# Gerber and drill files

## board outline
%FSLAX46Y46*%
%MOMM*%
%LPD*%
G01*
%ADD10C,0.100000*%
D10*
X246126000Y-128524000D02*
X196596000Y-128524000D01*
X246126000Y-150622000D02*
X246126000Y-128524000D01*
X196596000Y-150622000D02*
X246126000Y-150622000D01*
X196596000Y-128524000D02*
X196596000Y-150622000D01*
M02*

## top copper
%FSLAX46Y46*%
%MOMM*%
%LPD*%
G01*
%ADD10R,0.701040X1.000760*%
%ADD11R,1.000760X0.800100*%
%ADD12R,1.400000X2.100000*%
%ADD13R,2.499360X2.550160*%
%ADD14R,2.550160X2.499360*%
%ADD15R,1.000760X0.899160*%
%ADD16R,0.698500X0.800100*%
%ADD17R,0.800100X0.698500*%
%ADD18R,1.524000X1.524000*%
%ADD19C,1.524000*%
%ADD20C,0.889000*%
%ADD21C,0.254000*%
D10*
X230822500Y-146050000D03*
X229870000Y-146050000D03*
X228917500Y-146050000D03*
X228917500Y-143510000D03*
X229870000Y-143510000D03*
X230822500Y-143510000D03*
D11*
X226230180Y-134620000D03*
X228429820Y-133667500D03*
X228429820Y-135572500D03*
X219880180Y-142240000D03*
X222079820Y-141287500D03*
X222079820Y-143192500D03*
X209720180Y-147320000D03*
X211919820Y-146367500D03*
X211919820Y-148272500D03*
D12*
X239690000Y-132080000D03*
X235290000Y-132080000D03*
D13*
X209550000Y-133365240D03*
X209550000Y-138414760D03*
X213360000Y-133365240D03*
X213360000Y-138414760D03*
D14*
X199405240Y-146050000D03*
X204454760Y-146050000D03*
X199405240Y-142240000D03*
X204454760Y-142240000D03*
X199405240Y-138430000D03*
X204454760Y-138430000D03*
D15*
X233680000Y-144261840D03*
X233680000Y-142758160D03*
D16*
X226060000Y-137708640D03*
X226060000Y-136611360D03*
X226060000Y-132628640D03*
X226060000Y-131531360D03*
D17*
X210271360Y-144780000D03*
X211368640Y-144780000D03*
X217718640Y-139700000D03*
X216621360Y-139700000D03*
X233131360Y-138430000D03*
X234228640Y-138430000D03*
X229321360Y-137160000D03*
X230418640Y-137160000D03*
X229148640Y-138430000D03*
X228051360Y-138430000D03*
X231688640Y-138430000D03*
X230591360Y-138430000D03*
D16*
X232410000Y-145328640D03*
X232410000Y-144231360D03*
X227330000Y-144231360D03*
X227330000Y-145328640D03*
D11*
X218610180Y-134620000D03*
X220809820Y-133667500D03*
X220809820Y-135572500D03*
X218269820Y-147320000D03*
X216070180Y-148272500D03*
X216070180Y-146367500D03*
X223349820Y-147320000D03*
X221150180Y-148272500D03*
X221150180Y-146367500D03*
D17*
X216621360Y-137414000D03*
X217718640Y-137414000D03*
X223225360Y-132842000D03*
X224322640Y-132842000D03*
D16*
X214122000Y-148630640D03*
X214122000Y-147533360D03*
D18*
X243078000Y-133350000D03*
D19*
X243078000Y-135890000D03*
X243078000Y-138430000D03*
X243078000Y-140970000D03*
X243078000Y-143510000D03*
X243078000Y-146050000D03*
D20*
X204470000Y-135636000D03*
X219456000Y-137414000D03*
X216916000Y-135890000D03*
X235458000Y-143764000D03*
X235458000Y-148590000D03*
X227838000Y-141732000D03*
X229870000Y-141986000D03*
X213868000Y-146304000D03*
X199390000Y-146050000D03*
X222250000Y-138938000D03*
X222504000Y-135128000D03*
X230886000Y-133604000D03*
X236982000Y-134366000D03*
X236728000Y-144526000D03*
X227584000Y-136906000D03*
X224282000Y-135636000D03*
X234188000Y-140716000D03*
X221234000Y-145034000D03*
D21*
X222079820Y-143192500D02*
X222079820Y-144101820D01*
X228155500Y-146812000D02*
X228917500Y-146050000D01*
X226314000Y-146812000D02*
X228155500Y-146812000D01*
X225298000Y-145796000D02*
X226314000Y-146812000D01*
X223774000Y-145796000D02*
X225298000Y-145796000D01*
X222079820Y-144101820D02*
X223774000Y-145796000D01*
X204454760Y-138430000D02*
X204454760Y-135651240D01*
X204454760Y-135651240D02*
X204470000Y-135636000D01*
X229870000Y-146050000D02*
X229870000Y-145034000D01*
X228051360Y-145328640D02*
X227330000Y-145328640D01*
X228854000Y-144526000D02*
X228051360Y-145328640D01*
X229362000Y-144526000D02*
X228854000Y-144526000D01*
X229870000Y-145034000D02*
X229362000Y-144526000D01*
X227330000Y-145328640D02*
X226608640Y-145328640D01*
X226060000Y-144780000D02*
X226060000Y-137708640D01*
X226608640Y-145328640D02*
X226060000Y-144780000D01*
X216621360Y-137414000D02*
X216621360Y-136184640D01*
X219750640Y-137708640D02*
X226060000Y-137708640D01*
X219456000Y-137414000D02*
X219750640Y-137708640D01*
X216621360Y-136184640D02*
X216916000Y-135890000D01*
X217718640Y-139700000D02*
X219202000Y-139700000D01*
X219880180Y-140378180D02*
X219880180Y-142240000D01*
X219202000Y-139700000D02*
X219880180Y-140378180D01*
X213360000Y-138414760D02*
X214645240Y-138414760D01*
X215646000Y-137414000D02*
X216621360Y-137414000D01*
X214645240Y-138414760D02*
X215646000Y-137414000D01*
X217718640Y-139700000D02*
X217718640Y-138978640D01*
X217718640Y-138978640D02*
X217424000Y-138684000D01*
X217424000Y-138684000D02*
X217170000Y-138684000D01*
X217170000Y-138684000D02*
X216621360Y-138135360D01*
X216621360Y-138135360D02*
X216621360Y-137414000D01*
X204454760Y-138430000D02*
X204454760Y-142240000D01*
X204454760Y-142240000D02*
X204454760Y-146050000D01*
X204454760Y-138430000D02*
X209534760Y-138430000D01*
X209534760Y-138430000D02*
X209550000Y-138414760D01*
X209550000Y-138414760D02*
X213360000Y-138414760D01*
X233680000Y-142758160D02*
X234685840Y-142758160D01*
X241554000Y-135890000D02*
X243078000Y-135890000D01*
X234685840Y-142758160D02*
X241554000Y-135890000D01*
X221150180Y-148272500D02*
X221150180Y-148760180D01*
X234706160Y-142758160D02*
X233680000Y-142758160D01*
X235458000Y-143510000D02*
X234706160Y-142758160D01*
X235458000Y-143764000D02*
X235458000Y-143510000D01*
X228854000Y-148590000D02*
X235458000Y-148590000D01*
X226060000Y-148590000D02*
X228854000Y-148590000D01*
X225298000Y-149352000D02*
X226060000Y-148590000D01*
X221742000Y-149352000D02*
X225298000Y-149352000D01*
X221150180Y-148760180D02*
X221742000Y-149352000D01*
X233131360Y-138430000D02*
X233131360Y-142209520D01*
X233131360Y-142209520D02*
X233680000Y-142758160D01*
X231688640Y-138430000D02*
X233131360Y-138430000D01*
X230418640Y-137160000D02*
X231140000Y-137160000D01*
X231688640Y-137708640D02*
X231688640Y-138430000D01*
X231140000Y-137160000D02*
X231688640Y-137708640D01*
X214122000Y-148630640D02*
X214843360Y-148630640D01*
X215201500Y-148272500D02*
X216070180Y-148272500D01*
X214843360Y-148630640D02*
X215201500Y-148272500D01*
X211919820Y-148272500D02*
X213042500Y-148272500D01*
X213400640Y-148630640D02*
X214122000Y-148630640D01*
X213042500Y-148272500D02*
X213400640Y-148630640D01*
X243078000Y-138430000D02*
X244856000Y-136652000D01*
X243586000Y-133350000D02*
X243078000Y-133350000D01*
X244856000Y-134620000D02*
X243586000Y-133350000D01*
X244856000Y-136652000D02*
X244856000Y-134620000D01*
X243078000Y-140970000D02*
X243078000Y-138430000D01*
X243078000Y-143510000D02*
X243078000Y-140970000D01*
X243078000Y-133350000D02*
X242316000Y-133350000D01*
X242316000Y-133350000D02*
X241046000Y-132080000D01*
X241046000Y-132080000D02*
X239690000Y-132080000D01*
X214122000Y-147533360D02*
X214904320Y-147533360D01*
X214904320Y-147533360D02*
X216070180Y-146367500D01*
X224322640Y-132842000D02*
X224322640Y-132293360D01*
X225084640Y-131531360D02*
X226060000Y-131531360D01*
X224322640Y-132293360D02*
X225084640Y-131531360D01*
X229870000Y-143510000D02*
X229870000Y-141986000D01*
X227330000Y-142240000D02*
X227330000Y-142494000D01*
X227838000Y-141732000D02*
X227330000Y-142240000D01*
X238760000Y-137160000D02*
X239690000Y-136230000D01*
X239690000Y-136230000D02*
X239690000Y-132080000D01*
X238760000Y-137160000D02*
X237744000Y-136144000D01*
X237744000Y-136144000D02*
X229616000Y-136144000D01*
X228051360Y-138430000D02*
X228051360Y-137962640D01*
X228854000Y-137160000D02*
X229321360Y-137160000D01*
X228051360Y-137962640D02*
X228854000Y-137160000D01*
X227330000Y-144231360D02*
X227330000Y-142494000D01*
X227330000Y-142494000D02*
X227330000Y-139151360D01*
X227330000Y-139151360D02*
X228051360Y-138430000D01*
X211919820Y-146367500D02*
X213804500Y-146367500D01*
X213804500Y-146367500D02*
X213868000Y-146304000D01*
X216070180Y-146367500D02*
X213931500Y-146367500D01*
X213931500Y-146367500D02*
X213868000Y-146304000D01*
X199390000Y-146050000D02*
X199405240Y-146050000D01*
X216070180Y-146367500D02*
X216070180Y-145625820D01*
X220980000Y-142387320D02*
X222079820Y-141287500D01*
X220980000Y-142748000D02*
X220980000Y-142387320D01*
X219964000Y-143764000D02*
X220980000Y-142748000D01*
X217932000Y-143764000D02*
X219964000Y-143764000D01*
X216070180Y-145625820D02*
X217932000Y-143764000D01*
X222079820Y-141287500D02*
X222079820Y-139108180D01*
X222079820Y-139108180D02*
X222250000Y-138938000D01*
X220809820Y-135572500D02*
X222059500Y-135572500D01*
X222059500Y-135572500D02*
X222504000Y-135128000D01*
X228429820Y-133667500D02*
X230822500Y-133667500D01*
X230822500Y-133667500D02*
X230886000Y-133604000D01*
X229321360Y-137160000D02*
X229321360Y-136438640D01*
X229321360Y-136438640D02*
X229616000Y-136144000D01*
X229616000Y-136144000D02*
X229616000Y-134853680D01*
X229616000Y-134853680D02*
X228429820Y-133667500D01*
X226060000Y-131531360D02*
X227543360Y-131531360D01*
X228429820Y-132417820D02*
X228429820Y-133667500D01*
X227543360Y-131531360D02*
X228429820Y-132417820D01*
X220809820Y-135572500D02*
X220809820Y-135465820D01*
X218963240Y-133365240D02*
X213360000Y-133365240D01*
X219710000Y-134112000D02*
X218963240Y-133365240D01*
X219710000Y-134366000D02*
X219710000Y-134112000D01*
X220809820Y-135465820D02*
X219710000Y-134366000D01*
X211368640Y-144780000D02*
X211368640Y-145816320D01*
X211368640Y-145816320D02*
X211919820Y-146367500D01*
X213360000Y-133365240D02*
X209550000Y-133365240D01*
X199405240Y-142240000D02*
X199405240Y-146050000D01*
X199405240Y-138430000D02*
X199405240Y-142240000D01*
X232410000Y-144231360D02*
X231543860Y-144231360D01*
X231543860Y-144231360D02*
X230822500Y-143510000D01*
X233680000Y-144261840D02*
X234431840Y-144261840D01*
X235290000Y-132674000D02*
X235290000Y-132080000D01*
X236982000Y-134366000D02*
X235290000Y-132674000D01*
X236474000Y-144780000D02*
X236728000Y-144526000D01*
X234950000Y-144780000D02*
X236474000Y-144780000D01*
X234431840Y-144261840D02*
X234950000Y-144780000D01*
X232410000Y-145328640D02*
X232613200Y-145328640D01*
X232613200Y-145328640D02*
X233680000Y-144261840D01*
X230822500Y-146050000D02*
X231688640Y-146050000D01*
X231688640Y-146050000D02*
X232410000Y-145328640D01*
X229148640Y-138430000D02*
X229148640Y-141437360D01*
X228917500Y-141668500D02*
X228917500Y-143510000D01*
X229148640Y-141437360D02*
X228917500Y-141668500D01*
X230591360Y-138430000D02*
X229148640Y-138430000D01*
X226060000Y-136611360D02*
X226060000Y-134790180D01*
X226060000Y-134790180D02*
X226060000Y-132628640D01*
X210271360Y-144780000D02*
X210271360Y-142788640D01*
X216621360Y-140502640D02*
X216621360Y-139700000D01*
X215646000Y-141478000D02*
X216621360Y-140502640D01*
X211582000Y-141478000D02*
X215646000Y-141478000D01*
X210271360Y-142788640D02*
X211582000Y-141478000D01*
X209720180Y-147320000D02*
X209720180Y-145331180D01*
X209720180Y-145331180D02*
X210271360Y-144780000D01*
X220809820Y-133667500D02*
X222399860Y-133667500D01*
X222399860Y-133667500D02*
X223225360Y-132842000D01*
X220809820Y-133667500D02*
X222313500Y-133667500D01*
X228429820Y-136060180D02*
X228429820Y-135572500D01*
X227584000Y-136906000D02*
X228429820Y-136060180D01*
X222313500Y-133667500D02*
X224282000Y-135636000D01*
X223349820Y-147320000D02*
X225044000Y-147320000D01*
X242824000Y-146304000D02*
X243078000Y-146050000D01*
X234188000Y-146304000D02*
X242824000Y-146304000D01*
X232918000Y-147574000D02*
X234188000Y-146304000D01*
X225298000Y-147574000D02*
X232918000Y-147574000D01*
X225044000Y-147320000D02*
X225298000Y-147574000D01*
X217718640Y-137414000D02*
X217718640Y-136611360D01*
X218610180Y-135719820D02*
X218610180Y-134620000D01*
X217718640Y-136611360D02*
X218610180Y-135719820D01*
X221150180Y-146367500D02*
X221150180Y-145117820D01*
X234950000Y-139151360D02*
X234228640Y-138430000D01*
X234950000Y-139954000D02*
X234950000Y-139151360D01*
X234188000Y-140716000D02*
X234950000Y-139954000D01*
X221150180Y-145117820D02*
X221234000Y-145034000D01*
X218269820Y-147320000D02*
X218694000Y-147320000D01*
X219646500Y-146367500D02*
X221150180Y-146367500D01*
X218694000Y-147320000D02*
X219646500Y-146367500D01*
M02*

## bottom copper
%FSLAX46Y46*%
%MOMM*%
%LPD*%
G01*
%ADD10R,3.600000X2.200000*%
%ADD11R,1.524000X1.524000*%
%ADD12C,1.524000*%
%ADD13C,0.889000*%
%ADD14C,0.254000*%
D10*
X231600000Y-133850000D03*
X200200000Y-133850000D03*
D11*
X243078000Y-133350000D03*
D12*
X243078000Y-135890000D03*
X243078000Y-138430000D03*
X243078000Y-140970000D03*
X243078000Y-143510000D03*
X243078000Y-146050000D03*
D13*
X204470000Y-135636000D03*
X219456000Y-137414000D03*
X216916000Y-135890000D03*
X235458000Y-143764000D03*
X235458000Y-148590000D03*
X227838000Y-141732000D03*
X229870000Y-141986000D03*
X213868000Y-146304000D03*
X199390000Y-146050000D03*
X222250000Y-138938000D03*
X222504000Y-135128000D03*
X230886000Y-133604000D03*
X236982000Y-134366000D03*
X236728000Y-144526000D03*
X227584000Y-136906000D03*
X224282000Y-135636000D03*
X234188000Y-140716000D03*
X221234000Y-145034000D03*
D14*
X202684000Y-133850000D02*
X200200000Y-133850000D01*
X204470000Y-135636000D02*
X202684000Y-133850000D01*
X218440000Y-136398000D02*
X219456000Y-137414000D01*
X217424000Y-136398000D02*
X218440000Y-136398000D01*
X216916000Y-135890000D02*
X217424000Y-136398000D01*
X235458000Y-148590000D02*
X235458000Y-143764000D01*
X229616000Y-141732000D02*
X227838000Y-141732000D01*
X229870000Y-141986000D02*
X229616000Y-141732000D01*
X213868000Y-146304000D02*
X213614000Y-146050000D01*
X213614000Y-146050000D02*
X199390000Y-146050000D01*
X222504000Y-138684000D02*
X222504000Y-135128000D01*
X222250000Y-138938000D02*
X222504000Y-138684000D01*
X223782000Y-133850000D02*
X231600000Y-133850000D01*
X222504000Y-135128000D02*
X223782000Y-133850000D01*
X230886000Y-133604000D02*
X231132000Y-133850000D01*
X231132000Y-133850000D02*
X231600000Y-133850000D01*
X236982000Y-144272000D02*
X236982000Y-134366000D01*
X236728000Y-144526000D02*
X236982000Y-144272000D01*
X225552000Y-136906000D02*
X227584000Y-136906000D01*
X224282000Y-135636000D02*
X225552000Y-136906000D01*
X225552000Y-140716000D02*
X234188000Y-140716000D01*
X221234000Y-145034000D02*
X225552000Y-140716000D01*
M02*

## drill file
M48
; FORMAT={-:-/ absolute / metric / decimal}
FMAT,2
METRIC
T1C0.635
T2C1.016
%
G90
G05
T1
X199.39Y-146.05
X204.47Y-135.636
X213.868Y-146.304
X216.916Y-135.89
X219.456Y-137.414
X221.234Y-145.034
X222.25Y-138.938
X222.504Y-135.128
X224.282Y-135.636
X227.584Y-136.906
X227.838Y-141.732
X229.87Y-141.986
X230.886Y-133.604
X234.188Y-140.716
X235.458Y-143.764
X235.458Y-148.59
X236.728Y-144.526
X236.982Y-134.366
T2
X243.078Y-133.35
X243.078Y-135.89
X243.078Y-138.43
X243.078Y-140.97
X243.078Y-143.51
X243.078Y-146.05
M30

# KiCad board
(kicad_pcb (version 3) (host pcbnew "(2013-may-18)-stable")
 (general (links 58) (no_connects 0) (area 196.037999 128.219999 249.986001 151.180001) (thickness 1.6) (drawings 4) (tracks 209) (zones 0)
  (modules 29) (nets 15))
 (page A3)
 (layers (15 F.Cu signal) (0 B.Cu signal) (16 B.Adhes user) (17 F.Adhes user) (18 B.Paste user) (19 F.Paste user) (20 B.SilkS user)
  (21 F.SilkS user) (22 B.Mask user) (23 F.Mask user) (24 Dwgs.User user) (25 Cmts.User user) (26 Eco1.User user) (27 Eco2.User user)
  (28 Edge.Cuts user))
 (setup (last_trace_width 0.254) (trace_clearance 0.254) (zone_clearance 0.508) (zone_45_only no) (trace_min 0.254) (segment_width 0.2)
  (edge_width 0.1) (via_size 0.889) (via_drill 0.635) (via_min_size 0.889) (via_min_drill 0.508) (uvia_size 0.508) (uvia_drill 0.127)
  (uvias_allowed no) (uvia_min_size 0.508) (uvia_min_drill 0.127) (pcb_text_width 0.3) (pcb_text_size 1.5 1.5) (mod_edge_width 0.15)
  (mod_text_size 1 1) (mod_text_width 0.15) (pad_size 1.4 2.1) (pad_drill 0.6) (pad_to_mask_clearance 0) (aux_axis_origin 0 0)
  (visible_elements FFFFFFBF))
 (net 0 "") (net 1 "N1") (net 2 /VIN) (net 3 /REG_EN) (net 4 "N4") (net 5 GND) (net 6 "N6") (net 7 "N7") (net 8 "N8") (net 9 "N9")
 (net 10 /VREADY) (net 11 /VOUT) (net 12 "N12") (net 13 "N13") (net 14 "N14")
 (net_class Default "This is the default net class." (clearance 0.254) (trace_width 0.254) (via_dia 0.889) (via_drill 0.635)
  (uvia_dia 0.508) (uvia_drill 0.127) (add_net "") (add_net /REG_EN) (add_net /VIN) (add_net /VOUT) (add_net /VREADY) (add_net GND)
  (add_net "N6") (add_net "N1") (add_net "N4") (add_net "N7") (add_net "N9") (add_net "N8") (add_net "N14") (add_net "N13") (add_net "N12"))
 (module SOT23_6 (layer F.Cu) (at 229.87 144.78 180)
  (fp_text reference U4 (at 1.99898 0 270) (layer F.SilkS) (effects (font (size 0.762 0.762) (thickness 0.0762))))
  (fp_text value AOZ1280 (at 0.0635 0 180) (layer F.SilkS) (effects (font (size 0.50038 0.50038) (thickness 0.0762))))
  (pad 6 smd rect (at -0.9525 -1.27 180) (size 0.70104 1.00076) (layers F.Cu F.Paste F.Mask) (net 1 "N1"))
  (pad 5 smd rect (at 0 -1.27 180) (size 0.70104 1.00076) (layers F.Cu F.Paste F.Mask) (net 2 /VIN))
  (pad 4 smd rect (at 0.9525 -1.27 180) (size 0.70104 1.00076) (layers F.Cu F.Paste F.Mask) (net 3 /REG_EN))
  (pad 3 smd rect (at 0.9525 1.27 180) (size 0.70104 1.00076) (layers F.Cu F.Paste F.Mask) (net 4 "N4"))
  (pad 2 smd rect (at 0 1.27 180) (size 0.70104 1.00076) (layers F.Cu F.Paste F.Mask) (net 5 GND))
  (pad 1 smd rect (at -0.9525 1.27 180) (size 0.70104 1.00076) (layers F.Cu F.Paste F.Mask) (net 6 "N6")))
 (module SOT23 (layer F.Cu) (at 227.33 134.62 90)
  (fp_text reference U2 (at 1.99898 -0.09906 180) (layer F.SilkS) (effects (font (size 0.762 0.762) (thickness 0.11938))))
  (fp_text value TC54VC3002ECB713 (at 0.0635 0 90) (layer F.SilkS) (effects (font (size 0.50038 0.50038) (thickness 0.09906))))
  (pad 3 smd rect (at 0 -1.09982 90) (size 0.8001 1.00076) (layers F.Cu F.Paste F.Mask) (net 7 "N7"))
  (pad 2 smd rect (at 0.9525 1.09982 90) (size 0.8001 1.00076) (layers F.Cu F.Paste F.Mask) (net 5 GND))
  (pad 1 smd rect (at -0.9525 1.09982 90) (size 0.8001 1.00076) (layers F.Cu F.Paste F.Mask) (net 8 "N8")))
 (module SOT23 (layer F.Cu) (at 220.98 142.24 90)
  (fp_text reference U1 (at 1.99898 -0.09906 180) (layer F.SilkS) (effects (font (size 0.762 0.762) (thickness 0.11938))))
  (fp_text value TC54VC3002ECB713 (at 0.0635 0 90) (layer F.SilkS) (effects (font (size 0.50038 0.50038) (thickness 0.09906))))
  (pad 3 smd rect (at 0 -1.09982 90) (size 0.8001 1.00076) (layers F.Cu F.Paste F.Mask) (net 2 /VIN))
  (pad 2 smd rect (at 0.9525 1.09982 90) (size 0.8001 1.00076) (layers F.Cu F.Paste F.Mask) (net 5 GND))
  (pad 1 smd rect (at -0.9525 1.09982 90) (size 0.8001 1.00076) (layers F.Cu F.Paste F.Mask) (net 3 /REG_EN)))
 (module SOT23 (layer F.Cu) (at 210.82 147.32 90)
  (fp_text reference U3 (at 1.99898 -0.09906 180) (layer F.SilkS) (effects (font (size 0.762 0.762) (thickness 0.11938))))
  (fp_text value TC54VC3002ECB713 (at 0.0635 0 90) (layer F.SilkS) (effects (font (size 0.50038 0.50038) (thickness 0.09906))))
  (pad 3 smd rect (at 0 -1.09982 90) (size 0.8001 1.00076) (layers F.Cu F.Paste F.Mask) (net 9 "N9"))
  (pad 2 smd rect (at 0.9525 1.09982 90) (size 0.8001 1.00076) (layers F.Cu F.Paste F.Mask) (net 5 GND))
  (pad 1 smd rect (at -0.9525 1.09982 90) (size 0.8001 1.00076) (layers F.Cu F.Paste F.Mask) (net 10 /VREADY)))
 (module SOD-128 (layer F.Cu) (at 237.49 132.08 180)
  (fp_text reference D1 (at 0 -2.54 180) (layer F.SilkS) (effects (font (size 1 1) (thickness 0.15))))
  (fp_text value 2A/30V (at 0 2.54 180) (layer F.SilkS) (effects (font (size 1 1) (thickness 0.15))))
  (pad 1 smd rect (at -2.2 0 180) (size 1.4 2.1) (layers F.Cu F.Paste F.Mask) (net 5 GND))
  (pad 2 smd rect (at 2.2 0 180) (size 1.4 2.1) (layers F.Cu F.Paste F.Mask) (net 1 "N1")))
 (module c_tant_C (layer F.Cu) (at 209.55 135.89 90)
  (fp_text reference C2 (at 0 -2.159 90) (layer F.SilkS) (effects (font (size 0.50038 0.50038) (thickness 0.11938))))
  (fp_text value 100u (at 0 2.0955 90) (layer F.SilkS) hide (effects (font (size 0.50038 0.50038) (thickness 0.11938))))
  (pad 1 smd rect (at 2.52476 0 90) (size 2.55016 2.49936) (layers F.Cu F.Paste F.Mask) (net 5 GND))
  (pad 2 smd rect (at -2.52476 0 90) (size 2.55016 2.49936) (layers F.Cu F.Paste F.Mask) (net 2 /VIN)))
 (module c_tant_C (layer F.Cu) (at 213.36 135.89 90)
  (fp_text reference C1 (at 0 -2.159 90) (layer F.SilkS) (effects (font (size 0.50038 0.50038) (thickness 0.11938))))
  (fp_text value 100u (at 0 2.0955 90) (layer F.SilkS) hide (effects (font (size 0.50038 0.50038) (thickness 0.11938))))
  (pad 1 smd rect (at 2.52476 0 90) (size 2.55016 2.49936) (layers F.Cu F.Paste F.Mask) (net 5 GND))
  (pad 2 smd rect (at -2.52476 0 90) (size 2.55016 2.49936) (layers F.Cu F.Paste F.Mask) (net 2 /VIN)))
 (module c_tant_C (layer F.Cu) (at 201.93 146.05 180)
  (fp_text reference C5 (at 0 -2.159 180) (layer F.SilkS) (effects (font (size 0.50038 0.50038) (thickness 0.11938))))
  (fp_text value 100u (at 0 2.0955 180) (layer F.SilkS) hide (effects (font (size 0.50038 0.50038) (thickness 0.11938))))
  (pad 1 smd rect (at 2.52476 0 180) (size 2.55016 2.49936) (layers F.Cu F.Paste F.Mask) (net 5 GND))
  (pad 2 smd rect (at -2.52476 0 180) (size 2.55016 2.49936) (layers F.Cu F.Paste F.Mask) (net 2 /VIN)))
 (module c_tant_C (layer F.Cu) (at 201.93 142.24 180)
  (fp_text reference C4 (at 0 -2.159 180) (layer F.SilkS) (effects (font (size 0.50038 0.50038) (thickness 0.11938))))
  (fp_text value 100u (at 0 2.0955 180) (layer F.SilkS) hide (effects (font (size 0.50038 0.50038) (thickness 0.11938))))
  (pad 1 smd rect (at 2.52476 0 180) (size 2.55016 2.49936) (layers F.Cu F.Paste F.Mask) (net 5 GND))
  (pad 2 smd rect (at -2.52476 0 180) (size 2.55016 2.49936) (layers F.Cu F.Paste F.Mask) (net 2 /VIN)))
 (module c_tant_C (layer F.Cu) (at 201.93 138.43 180)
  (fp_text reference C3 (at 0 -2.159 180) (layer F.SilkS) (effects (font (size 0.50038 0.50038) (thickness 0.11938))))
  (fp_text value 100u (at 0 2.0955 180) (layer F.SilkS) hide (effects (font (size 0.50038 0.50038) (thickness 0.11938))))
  (pad 1 smd rect (at 2.52476 0 180) (size 2.55016 2.49936) (layers F.Cu F.Paste F.Mask) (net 5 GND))
  (pad 2 smd rect (at -2.52476 0 180) (size 2.55016 2.49936) (layers F.Cu F.Paste F.Mask) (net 2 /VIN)))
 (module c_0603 (layer F.Cu) (at 233.68 143.51 270)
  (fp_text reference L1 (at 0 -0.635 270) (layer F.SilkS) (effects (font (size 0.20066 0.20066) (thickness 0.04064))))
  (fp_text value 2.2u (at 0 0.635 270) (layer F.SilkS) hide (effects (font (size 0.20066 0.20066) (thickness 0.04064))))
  (pad 1 smd rect (at 0.75184 0 270) (size 0.89916 1.00076) (layers F.Cu F.Paste F.Mask) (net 1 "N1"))
  (pad 2 smd rect (at -0.75184 0 270) (size 0.89916 1.00076) (layers F.Cu F.Paste F.Mask) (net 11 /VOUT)))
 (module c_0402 (layer F.Cu) (at 226.06 137.16 270)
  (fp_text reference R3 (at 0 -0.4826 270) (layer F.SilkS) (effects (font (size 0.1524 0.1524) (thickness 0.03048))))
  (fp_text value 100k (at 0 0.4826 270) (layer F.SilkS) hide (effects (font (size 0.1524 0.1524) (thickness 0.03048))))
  (pad 1 smd rect (at 0.54864 0 270) (size 0.8001 0.6985) (layers F.Cu F.Paste F.Mask) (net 2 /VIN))
  (pad 2 smd rect (at -0.54864 0 270) (size 0.8001 0.6985) (layers F.Cu F.Paste F.Mask) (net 7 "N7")))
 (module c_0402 (layer F.Cu) (at 226.06 132.08 270)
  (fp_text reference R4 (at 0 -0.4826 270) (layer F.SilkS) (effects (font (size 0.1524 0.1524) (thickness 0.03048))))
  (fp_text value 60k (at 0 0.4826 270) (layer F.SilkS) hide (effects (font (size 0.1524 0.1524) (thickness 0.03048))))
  (pad 1 smd rect (at 0.54864 0 270) (size 0.8001 0.6985) (layers F.Cu F.Paste F.Mask) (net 7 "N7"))
  (pad 2 smd rect (at -0.54864 0 270) (size 0.8001 0.6985) (layers F.Cu F.Paste F.Mask) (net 5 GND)))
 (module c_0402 (layer F.Cu) (at 210.82 144.78 180)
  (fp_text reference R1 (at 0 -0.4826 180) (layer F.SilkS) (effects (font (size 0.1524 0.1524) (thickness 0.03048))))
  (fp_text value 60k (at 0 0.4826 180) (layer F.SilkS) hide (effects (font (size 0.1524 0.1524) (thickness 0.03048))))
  (pad 1 smd rect (at 0.54864 0 180) (size 0.8001 0.6985) (layers F.Cu F.Paste F.Mask) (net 9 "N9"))
  (pad 2 smd rect (at -0.54864 0 180) (size 0.8001 0.6985) (layers F.Cu F.Paste F.Mask) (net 5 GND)))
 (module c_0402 (layer F.Cu) (at 217.17 139.7)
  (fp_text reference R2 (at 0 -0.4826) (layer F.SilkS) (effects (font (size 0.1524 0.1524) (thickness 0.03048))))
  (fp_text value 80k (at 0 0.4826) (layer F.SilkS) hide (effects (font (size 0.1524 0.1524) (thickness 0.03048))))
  (pad 1 smd rect (at 0.54864 0) (size 0.8001 0.6985) (layers F.Cu F.Paste F.Mask) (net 2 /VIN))
  (pad 2 smd rect (at -0.54864 0) (size 0.8001 0.6985) (layers F.Cu F.Paste F.Mask) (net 9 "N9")))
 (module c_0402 (layer F.Cu) (at 233.68 138.43 180)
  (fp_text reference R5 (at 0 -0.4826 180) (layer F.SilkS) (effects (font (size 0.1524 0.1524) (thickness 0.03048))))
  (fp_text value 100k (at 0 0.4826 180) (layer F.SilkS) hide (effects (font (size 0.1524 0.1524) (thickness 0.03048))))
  (pad 1 smd rect (at 0.54864 0 180) (size 0.8001 0.6985) (layers F.Cu F.Paste F.Mask) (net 11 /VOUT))
  (pad 2 smd rect (at -0.54864 0 180) (size 0.8001 0.6985) (layers F.Cu F.Paste F.Mask) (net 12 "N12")))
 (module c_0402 (layer F.Cu) (at 229.87 137.16 180)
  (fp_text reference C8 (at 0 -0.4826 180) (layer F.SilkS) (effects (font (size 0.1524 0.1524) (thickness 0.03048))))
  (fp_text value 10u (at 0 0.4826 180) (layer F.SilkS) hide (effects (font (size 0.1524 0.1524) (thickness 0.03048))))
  (pad 1 smd rect (at 0.54864 0 180) (size 0.8001 0.6985) (layers F.Cu F.Paste F.Mask) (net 5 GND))
  (pad 2 smd rect (at -0.54864 0 180) (size 0.8001 0.6985) (layers F.Cu F.Paste F.Mask) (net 11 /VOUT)))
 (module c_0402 (layer F.Cu) (at 228.6 138.43)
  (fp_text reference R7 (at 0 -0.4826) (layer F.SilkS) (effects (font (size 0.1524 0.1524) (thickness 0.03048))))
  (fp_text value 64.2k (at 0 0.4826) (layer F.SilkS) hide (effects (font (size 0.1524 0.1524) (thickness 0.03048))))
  (pad 1 smd rect (at 0.54864 0) (size 0.8001 0.6985) (layers F.Cu F.Paste F.Mask) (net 4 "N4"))
  (pad 2 smd rect (at -0.54864 0) (size 0.8001 0.6985) (layers F.Cu F.Paste F.Mask) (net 5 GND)))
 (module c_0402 (layer F.Cu) (at 231.14 138.43)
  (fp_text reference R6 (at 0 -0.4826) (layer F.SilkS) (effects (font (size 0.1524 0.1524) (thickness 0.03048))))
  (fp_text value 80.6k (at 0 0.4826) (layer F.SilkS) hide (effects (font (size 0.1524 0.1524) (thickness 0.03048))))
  (pad 1 smd rect (at 0.54864 0) (size 0.8001 0.6985) (layers F.Cu F.Paste F.Mask) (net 11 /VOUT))
  (pad 2 smd rect (at -0.54864 0) (size 0.8001 0.6985) (layers F.Cu F.Paste F.Mask) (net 4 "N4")))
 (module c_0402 (layer F.Cu) (at 232.41 144.78 270)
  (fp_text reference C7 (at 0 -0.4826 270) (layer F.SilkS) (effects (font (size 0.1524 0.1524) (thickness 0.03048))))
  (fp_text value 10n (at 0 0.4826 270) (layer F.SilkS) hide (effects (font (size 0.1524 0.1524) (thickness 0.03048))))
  (pad 1 smd rect (at 0.54864 0 270) (size 0.8001 0.6985) (layers F.Cu F.Paste F.Mask) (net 1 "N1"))
  (pad 2 smd rect (at -0.54864 0 270) (size 0.8001 0.6985) (layers F.Cu F.Paste F.Mask) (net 6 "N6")))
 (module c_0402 (layer F.Cu) (at 227.33 144.78 90)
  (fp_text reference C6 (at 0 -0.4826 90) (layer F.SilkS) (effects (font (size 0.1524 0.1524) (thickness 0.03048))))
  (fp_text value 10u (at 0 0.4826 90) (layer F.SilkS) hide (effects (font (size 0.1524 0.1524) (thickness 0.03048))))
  (pad 1 smd rect (at 0.54864 0 90) (size 0.8001 0.6985) (layers F.Cu F.Paste F.Mask) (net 5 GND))
  (pad 2 smd rect (at -0.54864 0 90) (size 0.8001 0.6985) (layers F.Cu F.Paste F.Mask) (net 2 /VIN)))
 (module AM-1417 (layer B.Cu) (at 215.9 139.7)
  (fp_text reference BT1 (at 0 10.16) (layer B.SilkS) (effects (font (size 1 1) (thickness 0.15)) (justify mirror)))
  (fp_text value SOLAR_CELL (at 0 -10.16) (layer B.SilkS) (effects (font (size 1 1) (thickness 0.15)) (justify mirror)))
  (pad 2 smd rect (at 15.7 -5.85) (size 3.6 2.2) (layers B.Cu B.Paste B.Mask) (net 5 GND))
  (pad 1 smd rect (at -15.7 -5.85) (size 3.6 2.2) (layers B.Cu B.Paste B.Mask) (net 2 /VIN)))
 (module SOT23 (layer F.Cu) (at 219.71 134.62 90)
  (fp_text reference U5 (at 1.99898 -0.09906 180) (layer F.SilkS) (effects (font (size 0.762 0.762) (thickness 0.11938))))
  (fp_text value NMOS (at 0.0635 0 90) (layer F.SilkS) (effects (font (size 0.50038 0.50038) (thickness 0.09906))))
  (pad 3 smd rect (at 0 -1.09982 90) (size 0.8001 1.00076) (layers F.Cu F.Paste F.Mask) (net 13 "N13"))
  (pad 2 smd rect (at 0.9525 1.09982 90) (size 0.8001 1.00076) (layers F.Cu F.Paste F.Mask) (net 8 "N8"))
  (pad 1 smd rect (at -0.9525 1.09982 90) (size 0.8001 1.00076) (layers F.Cu F.Paste F.Mask) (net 5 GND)))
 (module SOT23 (layer F.Cu) (at 217.17 147.32 270)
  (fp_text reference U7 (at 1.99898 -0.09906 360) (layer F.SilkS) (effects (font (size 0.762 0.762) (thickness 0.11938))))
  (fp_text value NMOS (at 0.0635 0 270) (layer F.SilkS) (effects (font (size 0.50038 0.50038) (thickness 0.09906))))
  (pad 3 smd rect (at 0 -1.09982 270) (size 0.8001 1.00076) (layers F.Cu F.Paste F.Mask) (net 12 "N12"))
  (pad 2 smd rect (at 0.9525 1.09982 270) (size 0.8001 1.00076) (layers F.Cu F.Paste F.Mask) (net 10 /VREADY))
  (pad 1 smd rect (at -0.9525 1.09982 270) (size 0.8001 1.00076) (layers F.Cu F.Paste F.Mask) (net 5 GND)))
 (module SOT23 (layer F.Cu) (at 222.25 147.32 270)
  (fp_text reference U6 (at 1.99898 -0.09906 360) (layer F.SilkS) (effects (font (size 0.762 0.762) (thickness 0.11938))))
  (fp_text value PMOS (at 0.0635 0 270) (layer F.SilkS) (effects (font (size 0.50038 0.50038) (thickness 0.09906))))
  (pad 3 smd rect (at 0 -1.09982 270) (size 0.8001 1.00076) (layers F.Cu F.Paste F.Mask) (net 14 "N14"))
  (pad 2 smd rect (at 0.9525 1.09982 270) (size 0.8001 1.00076) (layers F.Cu F.Paste F.Mask) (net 11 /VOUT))
  (pad 1 smd rect (at -0.9525 1.09982 270) (size 0.8001 1.00076) (layers F.Cu F.Paste F.Mask) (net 12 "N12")))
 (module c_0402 (layer F.Cu) (at 217.17 137.414 180)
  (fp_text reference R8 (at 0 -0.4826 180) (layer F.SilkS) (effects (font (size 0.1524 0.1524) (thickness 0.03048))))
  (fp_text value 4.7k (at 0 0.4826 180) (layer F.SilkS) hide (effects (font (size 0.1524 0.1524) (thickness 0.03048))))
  (pad 1 smd rect (at 0.54864 0 180) (size 0.8001 0.6985) (layers F.Cu F.Paste F.Mask) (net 2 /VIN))
  (pad 2 smd rect (at -0.54864 0 180) (size 0.8001 0.6985) (layers F.Cu F.Paste F.Mask) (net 13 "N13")))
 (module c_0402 (layer F.Cu) (at 223.774 132.842 180)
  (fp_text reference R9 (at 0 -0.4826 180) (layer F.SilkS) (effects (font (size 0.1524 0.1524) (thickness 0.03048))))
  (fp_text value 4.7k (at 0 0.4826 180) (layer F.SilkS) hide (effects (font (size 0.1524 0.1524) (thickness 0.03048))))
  (pad 1 smd rect (at 0.54864 0 180) (size 0.8001 0.6985) (layers F.Cu F.Paste F.Mask) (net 8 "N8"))
  (pad 2 smd rect (at -0.54864 0 180) (size 0.8001 0.6985) (layers F.Cu F.Paste F.Mask) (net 5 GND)))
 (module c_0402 (layer F.Cu) (at 214.122 148.082 270)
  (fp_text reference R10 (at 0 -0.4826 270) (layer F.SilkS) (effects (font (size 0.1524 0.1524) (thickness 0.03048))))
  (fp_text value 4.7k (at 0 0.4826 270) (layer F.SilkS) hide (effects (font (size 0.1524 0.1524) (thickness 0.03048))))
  (pad 1 smd rect (at 0.54864 0 270) (size 0.8001 0.6985) (layers F.Cu F.Paste F.Mask) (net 10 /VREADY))
  (pad 2 smd rect (at -0.54864 0 270) (size 0.8001 0.6985) (layers F.Cu F.Paste F.Mask) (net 5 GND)))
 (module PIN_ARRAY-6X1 (layer F.Cu) (at 243.078 139.7 270)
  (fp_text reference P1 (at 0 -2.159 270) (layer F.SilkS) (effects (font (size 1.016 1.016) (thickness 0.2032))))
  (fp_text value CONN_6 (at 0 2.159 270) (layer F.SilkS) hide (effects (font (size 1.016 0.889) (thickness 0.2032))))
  (pad 1 thru_hole rect (at -6.35 0 270) (size 1.524 1.524) (drill 1.016) (layers *.Cu *.Mask F.SilkS) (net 5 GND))
  (pad 2 thru_hole circle (at -3.81 0 270) (size 1.524 1.524) (drill 1.016) (layers *.Cu *.Mask F.SilkS) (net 11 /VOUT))
  (pad 3 thru_hole circle (at -1.27 0 270) (size 1.524 1.524) (drill 1.016) (layers *.Cu *.Mask F.SilkS) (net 5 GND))
  (pad 4 thru_hole circle (at 1.27 0 270) (size 1.524 1.524) (drill 1.016) (layers *.Cu *.Mask F.SilkS) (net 5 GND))
  (pad 5 thru_hole circle (at 3.81 0 270) (size 1.524 1.524) (drill 1.016) (layers *.Cu *.Mask F.SilkS) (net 5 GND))
  (pad 6 thru_hole circle (at 6.35 0 270) (size 1.524 1.524) (drill 1.016) (layers *.Cu *.Mask F.SilkS) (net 14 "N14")))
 (gr_line (start 246.126 128.524) (end 196.596 128.524) (angle 90) (layer Edge.Cuts) (width 0.1))
 (gr_line (start 246.126 150.622) (end 246.126 128.524) (angle 90) (layer Edge.Cuts) (width 0.1))
 (gr_line (start 196.596 150.622) (end 246.126 150.622) (angle 90) (layer Edge.Cuts) (width 0.1))
 (gr_line (start 196.596 128.524) (end 196.596 150.622) (angle 90) (layer Edge.Cuts) (width 0.1))
 (segment (start 222.07982 143.1925) (end 222.07982 144.10182) (width 0.254) (layer F.Cu) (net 3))
 (segment (start 228.1555 146.812) (end 228.9175 146.05) (width 0.254) (layer F.Cu) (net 3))
 (segment (start 226.314 146.812) (end 228.1555 146.812) (width 0.254) (layer F.Cu) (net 3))
 (segment (start 225.298 145.796) (end 226.314 146.812) (width 0.254) (layer F.Cu) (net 3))
 (segment (start 223.774 145.796) (end 225.298 145.796) (width 0.254) (layer F.Cu) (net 3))
 (segment (start 222.07982 144.10182) (end 223.774 145.796) (width 0.254) (layer F.Cu) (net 3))
 (segment (start 204.45476 138.43) (end 204.45476 135.65124) (width 0.254) (layer F.Cu) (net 2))
 (segment (start 202.684 133.85) (end 200.2 133.85) (width 0.254) (layer B.Cu) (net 2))
 (segment (start 204.47 135.636) (end 202.684 133.85) (width 0.254) (layer B.Cu) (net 2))
 (via (at 204.47 135.636) (size 0.889) (layers F.Cu B.Cu) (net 2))
 (segment (start 204.45476 135.65124) (end 204.47 135.636) (width 0.254) (layer F.Cu) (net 2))
 (segment (start 229.87 146.05) (end 229.87 145.034) (width 0.254) (layer F.Cu) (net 2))
 (segment (start 228.05136 145.32864) (end 227.33 145.32864) (width 0.254) (layer F.Cu) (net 2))
 (segment (start 228.854 144.526) (end 228.05136 145.32864) (width 0.254) (layer F.Cu) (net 2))
 (segment (start 229.362 144.526) (end 228.854 144.526) (width 0.254) (layer F.Cu) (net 2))
 (segment (start 229.87 145.034) (end 229.362 144.526) (width 0.254) (layer F.Cu) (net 2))
 (segment (start 227.33 145.32864) (end 226.60864 145.32864) (width 0.254) (layer F.Cu) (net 2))
 (segment (start 226.06 144.78) (end 226.06 137.70864) (width 0.254) (layer F.Cu) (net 2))
 (segment (start 226.60864 145.32864) (end 226.06 144.78) (width 0.254) (layer F.Cu) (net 2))
 (segment (start 216.62136 137.414) (end 216.62136 136.18464) (width 0.254) (layer F.Cu) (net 2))
 (segment (start 219.75064 137.70864) (end 226.06 137.70864) (width 0.254) (layer F.Cu) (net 2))
 (segment (start 219.456 137.414) (end 219.75064 137.70864) (width 0.254) (layer F.Cu) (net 2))
 (via (at 219.456 137.414) (size 0.889) (layers F.Cu B.Cu) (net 2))
 (segment (start 218.44 136.398) (end 219.456 137.414) (width 0.254) (layer B.Cu) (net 2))
 (segment (start 217.424 136.398) (end 218.44 136.398) (width 0.254) (layer B.Cu) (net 2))
 (segment (start 216.916 135.89) (end 217.424 136.398) (width 0.254) (layer B.Cu) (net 2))
 (via (at 216.916 135.89) (size 0.889) (layers F.Cu B.Cu) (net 2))
 (segment (start 216.62136 136.18464) (end 216.916 135.89) (width 0.254) (layer F.Cu) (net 2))
 (segment (start 217.71864 139.7) (end 219.202 139.7) (width 0.254) (layer F.Cu) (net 2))
 (segment (start 219.88018 140.37818) (end 219.88018 142.24) (width 0.254) (layer F.Cu) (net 2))
 (segment (start 219.202 139.7) (end 219.88018 140.37818) (width 0.254) (layer F.Cu) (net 2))
 (segment (start 213.36 138.41476) (end 214.64524 138.41476) (width 0.254) (layer F.Cu) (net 2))
 (segment (start 215.646 137.414) (end 216.62136 137.414) (width 0.254) (layer F.Cu) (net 2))
 (segment (start 214.64524 138.41476) (end 215.646 137.414) (width 0.254) (layer F.Cu) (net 2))
 (segment (start 217.71864 139.7) (end 217.71864 138.97864) (width 0.254) (layer F.Cu) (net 2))
 (segment (start 217.71864 138.97864) (end 217.424 138.684) (width 0.254) (layer F.Cu) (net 2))
 (segment (start 217.424 138.684) (end 217.17 138.684) (width 0.254) (layer F.Cu) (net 2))
 (segment (start 217.17 138.684) (end 216.62136 138.13536) (width 0.254) (layer F.Cu) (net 2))
 (segment (start 216.62136 138.13536) (end 216.62136 137.414) (width 0.254) (layer F.Cu) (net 2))
 (segment (start 204.45476 138.43) (end 204.45476 142.24) (width 0.254) (layer F.Cu) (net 2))
 (segment (start 204.45476 142.24) (end 204.45476 146.05) (width 0.254) (layer F.Cu) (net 2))
 (segment (start 204.45476 138.43) (end 209.53476 138.43) (width 0.254) (layer F.Cu) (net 2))
 (segment (start 209.53476 138.43) (end 209.55 138.41476) (width 0.254) (layer F.Cu) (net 2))
 (segment (start 209.55 138.41476) (end 213.36 138.41476) (width 0.254) (layer F.Cu) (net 2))
 (segment (start 233.68 142.75816) (end 234.68584 142.75816) (width 0.254) (layer F.Cu) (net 11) (status 400000))
 (segment (start 241.554 135.89) (end 243.078 135.89) (width 0.254) (layer F.Cu) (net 11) (status 800000))
 (segment (start 234.68584 142.75816) (end 241.554 135.89) (width 0.254) (layer F.Cu) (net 11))
 (segment (start 221.15018 148.2725) (end 221.15018 148.76018) (width 0.254) (layer F.Cu) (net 11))
 (segment (start 234.70616 142.75816) (end 233.68 142.75816) (width 0.254) (layer F.Cu) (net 11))
 (segment (start 235.458 143.51) (end 234.70616 142.75816) (width 0.254) (layer F.Cu) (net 11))
 (segment (start 235.458 143.764) (end 235.458 143.51) (width 0.254) (layer F.Cu) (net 11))
 (via (at 235.458 143.764) (size 0.889) (layers F.Cu B.Cu) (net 11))
 (segment (start 235.458 148.59) (end 235.458 143.764) (width 0.254) (layer B.Cu) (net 11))
 (via (at 235.458 148.59) (size 0.889) (layers F.Cu B.Cu) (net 11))
 (segment (start 228.854 148.59) (end 235.458 148.59) (width 0.254) (layer F.Cu) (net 11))
 (segment (start 226.06 148.59) (end 228.854 148.59) (width 0.254) (layer F.Cu) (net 11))
 (segment (start 225.298 149.352) (end 226.06 148.59) (width 0.254) (layer F.Cu) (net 11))
 (segment (start 221.742 149.352) (end 225.298 149.352) (width 0.254) (layer F.Cu) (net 11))
 (segment (start 221.15018 148.76018) (end 221.742 149.352) (width 0.254) (layer F.Cu) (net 11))
 (segment (start 233.13136 138.43) (end 233.13136 142.20952) (width 0.254) (layer F.Cu) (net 11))
 (segment (start 233.13136 142.20952) (end 233.68 142.75816) (width 0.254) (layer F.Cu) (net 11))
 (segment (start 231.68864 138.43) (end 233.13136 138.43) (width 0.254) (layer F.Cu) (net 11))
 (segment (start 230.41864 137.16) (end 231.14 137.16) (width 0.254) (layer F.Cu) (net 11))
 (segment (start 231.68864 137.70864) (end 231.68864 138.43) (width 0.254) (layer F.Cu) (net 11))
 (segment (start 231.14 137.16) (end 231.68864 137.70864) (width 0.254) (layer F.Cu) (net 11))
 (segment (start 214.122 148.63064) (end 214.84336 148.63064) (width 0.254) (layer F.Cu) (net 10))
 (segment (start 215.2015 148.2725) (end 216.07018 148.2725) (width 0.254) (layer F.Cu) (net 10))
 (segment (start 214.84336 148.63064) (end 215.2015 148.2725) (width 0.254) (layer F.Cu) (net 10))
 (segment (start 211.91982 148.2725) (end 213.0425 148.2725) (width 0.254) (layer F.Cu) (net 10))
 (segment (start 213.40064 148.63064) (end 214.122 148.63064) (width 0.254) (layer F.Cu) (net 10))
 (segment (start 213.0425 148.2725) (end 213.40064 148.63064) (width 0.254) (layer F.Cu) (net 10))
 (segment (start 243.078 138.43) (end 244.856 136.652) (width 0.254) (layer F.Cu) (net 5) (status 400000))
 (segment (start 243.586 133.35) (end 243.078 133.35) (width 0.254) (layer F.Cu) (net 5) (status C00000))
 (segment (start 244.856 134.62) (end 243.586 133.35) (width 0.254) (layer F.Cu) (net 5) (status 800000))
 (segment (start 244.856 136.652) (end 244.856 134.62) (width 0.254) (layer F.Cu) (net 5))
 (segment (start 243.078 140.97) (end 243.078 138.43) (width 0.254) (layer F.Cu) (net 5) (status C00000))
 (segment (start 243.078 143.51) (end 243.078 140.97) (width 0.254) (layer F.Cu) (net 5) (status C00000))
 (segment (start 243.078 133.35) (end 242.316 133.35) (width 0.254) (layer F.Cu) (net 5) (status C00000))
 (segment (start 242.316 133.35) (end 241.046 132.08) (width 0.254) (layer F.Cu) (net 5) (status 400000))
 (segment (start 241.046 132.08) (end 239.69 132.08) (width 0.254) (layer F.Cu) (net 5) (status 800000))
 (segment (start 214.122 147.53336) (end 214.90432 147.53336) (width 0.254) (layer F.Cu) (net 5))
 (segment (start 214.90432 147.53336) (end 216.07018 146.3675) (width 0.254) (layer F.Cu) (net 5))
 (segment (start 224.32264 132.842) (end 224.32264 132.29336) (width 0.254) (layer F.Cu) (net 5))
 (segment (start 225.08464 131.53136) (end 226.06 131.53136) (width 0.254) (layer F.Cu) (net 5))
 (segment (start 224.32264 132.29336) (end 225.08464 131.53136) (width 0.254) (layer F.Cu) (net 5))
 (segment (start 229.87 143.51) (end 229.87 141.986) (width 0.254) (layer F.Cu) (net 5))
 (segment (start 227.33 142.24) (end 227.33 142.494) (width 0.254) (layer F.Cu) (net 5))
 (segment (start 227.838 141.732) (end 227.33 142.24) (width 0.254) (layer F.Cu) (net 5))
 (via (at 227.838 141.732) (size 0.889) (layers F.Cu B.Cu) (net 5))
 (segment (start 229.616 141.732) (end 227.838 141.732) (width 0.254) (layer B.Cu) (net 5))
 (segment (start 229.87 141.986) (end 229.616 141.732) (width 0.254) (layer B.Cu) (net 5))
 (via (at 229.87 141.986) (size 0.889) (layers F.Cu B.Cu) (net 5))
 (segment (start 238.76 137.16) (end 239.69 136.23) (width 0.254) (layer F.Cu) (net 5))
 (segment (start 239.69 136.23) (end 239.69 132.08) (width 0.254) (layer F.Cu) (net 5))
 (segment (start 238.76 137.16) (end 237.744 136.144) (width 0.254) (layer F.Cu) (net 5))
 (segment (start 237.744 136.144) (end 229.616 136.144) (width 0.254) (layer F.Cu) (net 5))
 (segment (start 228.05136 138.43) (end 228.05136 137.96264) (width 0.254) (layer F.Cu) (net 5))
 (segment (start 228.854 137.16) (end 229.32136 137.16) (width 0.254) (layer F.Cu) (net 5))
 (segment (start 228.05136 137.96264) (end 228.854 137.16) (width 0.254) (layer F.Cu) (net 5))
 (segment (start 227.33 144.23136) (end 227.33 142.494) (width 0.254) (layer F.Cu) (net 5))
 (segment (start 227.33 142.494) (end 227.33 139.15136) (width 0.254) (layer F.Cu) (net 5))
 (segment (start 227.33 139.15136) (end 228.05136 138.43) (width 0.254) (layer F.Cu) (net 5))
 (segment (start 211.91982 146.3675) (end 213.8045 146.3675) (width 0.254) (layer F.Cu) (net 5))
 (segment (start 213.8045 146.3675) (end 213.868 146.304) (width 0.254) (layer F.Cu) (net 5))
 (segment (start 216.07018 146.3675) (end 213.9315 146.3675) (width 0.254) (layer F.Cu) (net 5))
 (segment (start 213.9315 146.3675) (end 213.868 146.304) (width 0.254) (layer F.Cu) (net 5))
 (segment (start 199.39 146.05) (end 199.40524 146.05) (width 0.254) (layer F.Cu) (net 5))
 (via (at 213.868 146.304) (size 0.889) (layers F.Cu B.Cu) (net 5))
 (segment (start 213.868 146.304) (end 213.614 146.05) (width 0.254) (layer B.Cu) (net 5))
 (segment (start 213.614 146.05) (end 199.39 146.05) (width 0.254) (layer B.Cu) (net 5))
 (via (at 199.39 146.05) (size 0.889) (layers F.Cu B.Cu) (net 5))
 (segment (start 216.07018 146.3675) (end 216.07018 145.62582) (width 0.254) (layer F.Cu) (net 5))
 (segment (start 220.98 142.38732) (end 222.07982 141.2875) (width 0.254) (layer F.Cu) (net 5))
 (segment (start 220.98 142.748) (end 220.98 142.38732) (width 0.254) (layer F.Cu) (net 5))
 (segment (start 219.964 143.764) (end 220.98 142.748) (width 0.254) (layer F.Cu) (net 5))
 (segment (start 217.932 143.764) (end 219.964 143.764) (width 0.254) (layer F.Cu) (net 5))
 (segment (start 216.07018 145.62582) (end 217.932 143.764) (width 0.254) (layer F.Cu) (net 5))
 (segment (start 222.07982 141.2875) (end 222.07982 139.10818) (width 0.254) (layer F.Cu) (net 5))
 (segment (start 222.504 138.684) (end 222.504 135.128) (width 0.254) (layer B.Cu) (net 5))
 (segment (start 222.25 138.938) (end 222.504 138.684) (width 0.254) (layer B.Cu) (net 5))
 (via (at 222.25 138.938) (size 0.889) (layers F.Cu B.Cu) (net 5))
 (segment (start 222.07982 139.10818) (end 222.25 138.938) (width 0.254) (layer F.Cu) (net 5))
 (segment (start 220.80982 135.5725) (end 222.0595 135.5725) (width 0.254) (layer F.Cu) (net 5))
 (segment (start 223.782 133.85) (end 231.6 133.85) (width 0.254) (layer B.Cu) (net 5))
 (segment (start 222.504 135.128) (end 223.782 133.85) (width 0.254) (layer B.Cu) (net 5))
 (via (at 222.504 135.128) (size 0.889) (layers F.Cu B.Cu) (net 5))
 (segment (start 222.0595 135.5725) (end 222.504 135.128) (width 0.254) (layer F.Cu) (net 5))
 (segment (start 228.42982 133.6675) (end 230.8225 133.6675) (width 0.254) (layer F.Cu) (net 5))
 (segment (start 230.8225 133.6675) (end 230.886 133.604) (width 0.254) (layer F.Cu) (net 5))
 (via (at 230.886 133.604) (size 0.889) (layers F.Cu B.Cu) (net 5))
 (segment (start 230.886 133.604) (end 231.132 133.85) (width 0.254) (layer B.Cu) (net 5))
 (segment (start 231.132 133.85) (end 231.6 133.85) (width 0.254) (layer B.Cu) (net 5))
 (segment (start 229.32136 137.16) (end 229.32136 136.43864) (width 0.254) (layer F.Cu) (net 5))
 (segment (start 229.32136 136.43864) (end 229.616 136.144) (width 0.254) (layer F.Cu) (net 5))
 (segment (start 229.616 136.144) (end 229.616 134.85368) (width 0.254) (layer F.Cu) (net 5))
 (segment (start 229.616 134.85368) (end 228.42982 133.6675) (width 0.254) (layer F.Cu) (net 5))
 (segment (start 226.06 131.53136) (end 227.54336 131.53136) (width 0.254) (layer F.Cu) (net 5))
 (segment (start 228.42982 132.41782) (end 228.42982 133.6675) (width 0.254) (layer F.Cu) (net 5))
 (segment (start 227.54336 131.53136) (end 228.42982 132.41782) (width 0.254) (layer F.Cu) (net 5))
 (segment (start 220.80982 135.5725) (end 220.80982 135.46582) (width 0.254) (layer F.Cu) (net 5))
 (segment (start 218.96324 133.36524) (end 213.36 133.36524) (width 0.254) (layer F.Cu) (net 5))
 (segment (start 219.71 134.112) (end 218.96324 133.36524) (width 0.254) (layer F.Cu) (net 5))
 (segment (start 219.71 134.366) (end 219.71 134.112) (width 0.254) (layer F.Cu) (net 5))
 (segment (start 220.80982 135.46582) (end 219.71 134.366) (width 0.254) (layer F.Cu) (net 5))
 (segment (start 211.36864 144.78) (end 211.36864 145.81632) (width 0.254) (layer F.Cu) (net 5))
 (segment (start 211.36864 145.81632) (end 211.91982 146.3675) (width 0.254) (layer F.Cu) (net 5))
 (segment (start 213.36 133.36524) (end 209.55 133.36524) (width 0.254) (layer F.Cu) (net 5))
 (segment (start 199.40524 142.24) (end 199.40524 146.05) (width 0.254) (layer F.Cu) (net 5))
 (segment (start 199.40524 138.43) (end 199.40524 142.24) (width 0.254) (layer F.Cu) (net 5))
 (segment (start 232.41 144.23136) (end 231.54386 144.23136) (width 0.254) (layer F.Cu) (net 6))
 (segment (start 231.54386 144.23136) (end 230.8225 143.51) (width 0.254) (layer F.Cu) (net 6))
 (segment (start 233.68 144.26184) (end 234.43184 144.26184) (width 0.254) (layer F.Cu) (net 1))
 (segment (start 235.29 132.674) (end 235.29 132.08) (width 0.254) (layer F.Cu) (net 1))
 (segment (start 236.982 134.366) (end 235.29 132.674) (width 0.254) (layer F.Cu) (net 1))
 (via (at 236.982 134.366) (size 0.889) (layers F.Cu B.Cu) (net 1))
 (segment (start 236.982 144.272) (end 236.982 134.366) (width 0.254) (layer B.Cu) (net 1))
 (segment (start 236.728 144.526) (end 236.982 144.272) (width 0.254) (layer B.Cu) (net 1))
 (via (at 236.728 144.526) (size 0.889) (layers F.Cu B.Cu) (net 1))
 (segment (start 236.474 144.78) (end 236.728 144.526) (width 0.254) (layer F.Cu) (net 1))
 (segment (start 234.95 144.78) (end 236.474 144.78) (width 0.254) (layer F.Cu) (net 1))
 (segment (start 234.43184 144.26184) (end 234.95 144.78) (width 0.254) (layer F.Cu) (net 1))
 (segment (start 232.41 145.32864) (end 232.6132 145.32864) (width 0.254) (layer F.Cu) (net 1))
 (segment (start 232.6132 145.32864) (end 233.68 144.26184) (width 0.254) (layer F.Cu) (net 1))
 (segment (start 230.8225 146.05) (end 231.68864 146.05) (width 0.254) (layer F.Cu) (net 1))
 (segment (start 231.68864 146.05) (end 232.41 145.32864) (width 0.254) (layer F.Cu) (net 1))
 (segment (start 229.14864 138.43) (end 229.14864 141.43736) (width 0.254) (layer F.Cu) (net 4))
 (segment (start 228.9175 141.6685) (end 228.9175 143.51) (width 0.254) (layer F.Cu) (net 4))
 (segment (start 229.14864 141.43736) (end 228.9175 141.6685) (width 0.254) (layer F.Cu) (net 4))
 (segment (start 230.59136 138.43) (end 229.14864 138.43) (width 0.254) (layer F.Cu) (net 4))
 (segment (start 226.06 136.61136) (end 226.06 134.79018) (width 0.254) (layer F.Cu) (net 7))
 (segment (start 226.06 134.79018) (end 226.06 132.62864) (width 0.254) (layer F.Cu) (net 7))
 (segment (start 210.27136 144.78) (end 210.27136 142.78864) (width 0.254) (layer F.Cu) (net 9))
 (segment (start 216.62136 140.50264) (end 216.62136 139.7) (width 0.254) (layer F.Cu) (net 9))
 (segment (start 215.646 141.478) (end 216.62136 140.50264) (width 0.254) (layer F.Cu) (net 9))
 (segment (start 211.582 141.478) (end 215.646 141.478) (width 0.254) (layer F.Cu) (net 9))
 (segment (start 210.27136 142.78864) (end 211.582 141.478) (width 0.254) (layer F.Cu) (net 9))
 (segment (start 209.72018 147.32) (end 209.72018 145.33118) (width 0.254) (layer F.Cu) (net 9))
 (segment (start 209.72018 145.33118) (end 210.27136 144.78) (width 0.254) (layer F.Cu) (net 9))
 (segment (start 220.80982 133.6675) (end 222.39986 133.6675) (width 0.254) (layer F.Cu) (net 8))
 (segment (start 222.39986 133.6675) (end 223.22536 132.842) (width 0.254) (layer F.Cu) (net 8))
 (segment (start 220.80982 133.6675) (end 222.3135 133.6675) (width 0.254) (layer F.Cu) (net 8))
 (segment (start 228.42982 136.06018) (end 228.42982 135.5725) (width 0.254) (layer F.Cu) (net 8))
 (segment (start 227.584 136.906) (end 228.42982 136.06018) (width 0.254) (layer F.Cu) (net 8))
 (via (at 227.584 136.906) (size 0.889) (layers F.Cu B.Cu) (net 8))
 (segment (start 225.552 136.906) (end 227.584 136.906) (width 0.254) (layer B.Cu) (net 8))
 (segment (start 224.282 135.636) (end 225.552 136.906) (width 0.254) (layer B.Cu) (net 8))
 (via (at 224.282 135.636) (size 0.889) (layers F.Cu B.Cu) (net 8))
 (segment (start 222.3135 133.6675) (end 224.282 135.636) (width 0.254) (layer F.Cu) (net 8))
 (segment (start 223.34982 147.32) (end 225.044 147.32) (width 0.254) (layer F.Cu) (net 14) (status 400000))
 (segment (start 242.824 146.304) (end 243.078 146.05) (width 0.254) (layer F.Cu) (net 14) (status C00000))
 (segment (start 234.188 146.304) (end 242.824 146.304) (width 0.254) (layer F.Cu) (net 14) (status 800000))
 (segment (start 232.918 147.574) (end 234.188 146.304) (width 0.254) (layer F.Cu) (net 14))
 (segment (start 225.298 147.574) (end 232.918 147.574) (width 0.254) (layer F.Cu) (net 14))
 (segment (start 225.044 147.32) (end 225.298 147.574) (width 0.254) (layer F.Cu) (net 14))
 (segment (start 217.71864 137.414) (end 217.71864 136.61136) (width 0.254) (layer F.Cu) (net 13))
 (segment (start 218.61018 135.71982) (end 218.61018 134.62) (width 0.254) (layer F.Cu) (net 13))
 (segment (start 217.71864 136.61136) (end 218.61018 135.71982) (width 0.254) (layer F.Cu) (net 13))
 (segment (start 221.15018 146.3675) (end 221.15018 145.11782) (width 0.254) (layer F.Cu) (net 12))
 (segment (start 234.95 139.15136) (end 234.22864 138.43) (width 0.254) (layer F.Cu) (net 12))
 (segment (start 234.95 139.954) (end 234.95 139.15136) (width 0.254) (layer F.Cu) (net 12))
 (segment (start 234.188 140.716) (end 234.95 139.954) (width 0.254) (layer F.Cu) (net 12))
 (via (at 234.188 140.716) (size 0.889) (layers F.Cu B.Cu) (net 12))
 (segment (start 225.552 140.716) (end 234.188 140.716) (width 0.254) (layer B.Cu) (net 12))
 (segment (start 221.234 145.034) (end 225.552 140.716) (width 0.254) (layer B.Cu) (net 12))
 (via (at 221.234 145.034) (size 0.889) (layers F.Cu B.Cu) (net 12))
 (segment (start 221.15018 145.11782) (end 221.234 145.034) (width 0.254) (layer F.Cu) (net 12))
 (segment (start 218.26982 147.32) (end 218.694 147.32) (width 0.254) (layer F.Cu) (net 12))
 (segment (start 219.6465 146.3675) (end 221.15018 146.3675) (width 0.254) (layer F.Cu) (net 12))
 (segment (start 218.694 147.32) (end 219.6465 146.3675) (width 0.254) (layer F.Cu) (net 12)))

